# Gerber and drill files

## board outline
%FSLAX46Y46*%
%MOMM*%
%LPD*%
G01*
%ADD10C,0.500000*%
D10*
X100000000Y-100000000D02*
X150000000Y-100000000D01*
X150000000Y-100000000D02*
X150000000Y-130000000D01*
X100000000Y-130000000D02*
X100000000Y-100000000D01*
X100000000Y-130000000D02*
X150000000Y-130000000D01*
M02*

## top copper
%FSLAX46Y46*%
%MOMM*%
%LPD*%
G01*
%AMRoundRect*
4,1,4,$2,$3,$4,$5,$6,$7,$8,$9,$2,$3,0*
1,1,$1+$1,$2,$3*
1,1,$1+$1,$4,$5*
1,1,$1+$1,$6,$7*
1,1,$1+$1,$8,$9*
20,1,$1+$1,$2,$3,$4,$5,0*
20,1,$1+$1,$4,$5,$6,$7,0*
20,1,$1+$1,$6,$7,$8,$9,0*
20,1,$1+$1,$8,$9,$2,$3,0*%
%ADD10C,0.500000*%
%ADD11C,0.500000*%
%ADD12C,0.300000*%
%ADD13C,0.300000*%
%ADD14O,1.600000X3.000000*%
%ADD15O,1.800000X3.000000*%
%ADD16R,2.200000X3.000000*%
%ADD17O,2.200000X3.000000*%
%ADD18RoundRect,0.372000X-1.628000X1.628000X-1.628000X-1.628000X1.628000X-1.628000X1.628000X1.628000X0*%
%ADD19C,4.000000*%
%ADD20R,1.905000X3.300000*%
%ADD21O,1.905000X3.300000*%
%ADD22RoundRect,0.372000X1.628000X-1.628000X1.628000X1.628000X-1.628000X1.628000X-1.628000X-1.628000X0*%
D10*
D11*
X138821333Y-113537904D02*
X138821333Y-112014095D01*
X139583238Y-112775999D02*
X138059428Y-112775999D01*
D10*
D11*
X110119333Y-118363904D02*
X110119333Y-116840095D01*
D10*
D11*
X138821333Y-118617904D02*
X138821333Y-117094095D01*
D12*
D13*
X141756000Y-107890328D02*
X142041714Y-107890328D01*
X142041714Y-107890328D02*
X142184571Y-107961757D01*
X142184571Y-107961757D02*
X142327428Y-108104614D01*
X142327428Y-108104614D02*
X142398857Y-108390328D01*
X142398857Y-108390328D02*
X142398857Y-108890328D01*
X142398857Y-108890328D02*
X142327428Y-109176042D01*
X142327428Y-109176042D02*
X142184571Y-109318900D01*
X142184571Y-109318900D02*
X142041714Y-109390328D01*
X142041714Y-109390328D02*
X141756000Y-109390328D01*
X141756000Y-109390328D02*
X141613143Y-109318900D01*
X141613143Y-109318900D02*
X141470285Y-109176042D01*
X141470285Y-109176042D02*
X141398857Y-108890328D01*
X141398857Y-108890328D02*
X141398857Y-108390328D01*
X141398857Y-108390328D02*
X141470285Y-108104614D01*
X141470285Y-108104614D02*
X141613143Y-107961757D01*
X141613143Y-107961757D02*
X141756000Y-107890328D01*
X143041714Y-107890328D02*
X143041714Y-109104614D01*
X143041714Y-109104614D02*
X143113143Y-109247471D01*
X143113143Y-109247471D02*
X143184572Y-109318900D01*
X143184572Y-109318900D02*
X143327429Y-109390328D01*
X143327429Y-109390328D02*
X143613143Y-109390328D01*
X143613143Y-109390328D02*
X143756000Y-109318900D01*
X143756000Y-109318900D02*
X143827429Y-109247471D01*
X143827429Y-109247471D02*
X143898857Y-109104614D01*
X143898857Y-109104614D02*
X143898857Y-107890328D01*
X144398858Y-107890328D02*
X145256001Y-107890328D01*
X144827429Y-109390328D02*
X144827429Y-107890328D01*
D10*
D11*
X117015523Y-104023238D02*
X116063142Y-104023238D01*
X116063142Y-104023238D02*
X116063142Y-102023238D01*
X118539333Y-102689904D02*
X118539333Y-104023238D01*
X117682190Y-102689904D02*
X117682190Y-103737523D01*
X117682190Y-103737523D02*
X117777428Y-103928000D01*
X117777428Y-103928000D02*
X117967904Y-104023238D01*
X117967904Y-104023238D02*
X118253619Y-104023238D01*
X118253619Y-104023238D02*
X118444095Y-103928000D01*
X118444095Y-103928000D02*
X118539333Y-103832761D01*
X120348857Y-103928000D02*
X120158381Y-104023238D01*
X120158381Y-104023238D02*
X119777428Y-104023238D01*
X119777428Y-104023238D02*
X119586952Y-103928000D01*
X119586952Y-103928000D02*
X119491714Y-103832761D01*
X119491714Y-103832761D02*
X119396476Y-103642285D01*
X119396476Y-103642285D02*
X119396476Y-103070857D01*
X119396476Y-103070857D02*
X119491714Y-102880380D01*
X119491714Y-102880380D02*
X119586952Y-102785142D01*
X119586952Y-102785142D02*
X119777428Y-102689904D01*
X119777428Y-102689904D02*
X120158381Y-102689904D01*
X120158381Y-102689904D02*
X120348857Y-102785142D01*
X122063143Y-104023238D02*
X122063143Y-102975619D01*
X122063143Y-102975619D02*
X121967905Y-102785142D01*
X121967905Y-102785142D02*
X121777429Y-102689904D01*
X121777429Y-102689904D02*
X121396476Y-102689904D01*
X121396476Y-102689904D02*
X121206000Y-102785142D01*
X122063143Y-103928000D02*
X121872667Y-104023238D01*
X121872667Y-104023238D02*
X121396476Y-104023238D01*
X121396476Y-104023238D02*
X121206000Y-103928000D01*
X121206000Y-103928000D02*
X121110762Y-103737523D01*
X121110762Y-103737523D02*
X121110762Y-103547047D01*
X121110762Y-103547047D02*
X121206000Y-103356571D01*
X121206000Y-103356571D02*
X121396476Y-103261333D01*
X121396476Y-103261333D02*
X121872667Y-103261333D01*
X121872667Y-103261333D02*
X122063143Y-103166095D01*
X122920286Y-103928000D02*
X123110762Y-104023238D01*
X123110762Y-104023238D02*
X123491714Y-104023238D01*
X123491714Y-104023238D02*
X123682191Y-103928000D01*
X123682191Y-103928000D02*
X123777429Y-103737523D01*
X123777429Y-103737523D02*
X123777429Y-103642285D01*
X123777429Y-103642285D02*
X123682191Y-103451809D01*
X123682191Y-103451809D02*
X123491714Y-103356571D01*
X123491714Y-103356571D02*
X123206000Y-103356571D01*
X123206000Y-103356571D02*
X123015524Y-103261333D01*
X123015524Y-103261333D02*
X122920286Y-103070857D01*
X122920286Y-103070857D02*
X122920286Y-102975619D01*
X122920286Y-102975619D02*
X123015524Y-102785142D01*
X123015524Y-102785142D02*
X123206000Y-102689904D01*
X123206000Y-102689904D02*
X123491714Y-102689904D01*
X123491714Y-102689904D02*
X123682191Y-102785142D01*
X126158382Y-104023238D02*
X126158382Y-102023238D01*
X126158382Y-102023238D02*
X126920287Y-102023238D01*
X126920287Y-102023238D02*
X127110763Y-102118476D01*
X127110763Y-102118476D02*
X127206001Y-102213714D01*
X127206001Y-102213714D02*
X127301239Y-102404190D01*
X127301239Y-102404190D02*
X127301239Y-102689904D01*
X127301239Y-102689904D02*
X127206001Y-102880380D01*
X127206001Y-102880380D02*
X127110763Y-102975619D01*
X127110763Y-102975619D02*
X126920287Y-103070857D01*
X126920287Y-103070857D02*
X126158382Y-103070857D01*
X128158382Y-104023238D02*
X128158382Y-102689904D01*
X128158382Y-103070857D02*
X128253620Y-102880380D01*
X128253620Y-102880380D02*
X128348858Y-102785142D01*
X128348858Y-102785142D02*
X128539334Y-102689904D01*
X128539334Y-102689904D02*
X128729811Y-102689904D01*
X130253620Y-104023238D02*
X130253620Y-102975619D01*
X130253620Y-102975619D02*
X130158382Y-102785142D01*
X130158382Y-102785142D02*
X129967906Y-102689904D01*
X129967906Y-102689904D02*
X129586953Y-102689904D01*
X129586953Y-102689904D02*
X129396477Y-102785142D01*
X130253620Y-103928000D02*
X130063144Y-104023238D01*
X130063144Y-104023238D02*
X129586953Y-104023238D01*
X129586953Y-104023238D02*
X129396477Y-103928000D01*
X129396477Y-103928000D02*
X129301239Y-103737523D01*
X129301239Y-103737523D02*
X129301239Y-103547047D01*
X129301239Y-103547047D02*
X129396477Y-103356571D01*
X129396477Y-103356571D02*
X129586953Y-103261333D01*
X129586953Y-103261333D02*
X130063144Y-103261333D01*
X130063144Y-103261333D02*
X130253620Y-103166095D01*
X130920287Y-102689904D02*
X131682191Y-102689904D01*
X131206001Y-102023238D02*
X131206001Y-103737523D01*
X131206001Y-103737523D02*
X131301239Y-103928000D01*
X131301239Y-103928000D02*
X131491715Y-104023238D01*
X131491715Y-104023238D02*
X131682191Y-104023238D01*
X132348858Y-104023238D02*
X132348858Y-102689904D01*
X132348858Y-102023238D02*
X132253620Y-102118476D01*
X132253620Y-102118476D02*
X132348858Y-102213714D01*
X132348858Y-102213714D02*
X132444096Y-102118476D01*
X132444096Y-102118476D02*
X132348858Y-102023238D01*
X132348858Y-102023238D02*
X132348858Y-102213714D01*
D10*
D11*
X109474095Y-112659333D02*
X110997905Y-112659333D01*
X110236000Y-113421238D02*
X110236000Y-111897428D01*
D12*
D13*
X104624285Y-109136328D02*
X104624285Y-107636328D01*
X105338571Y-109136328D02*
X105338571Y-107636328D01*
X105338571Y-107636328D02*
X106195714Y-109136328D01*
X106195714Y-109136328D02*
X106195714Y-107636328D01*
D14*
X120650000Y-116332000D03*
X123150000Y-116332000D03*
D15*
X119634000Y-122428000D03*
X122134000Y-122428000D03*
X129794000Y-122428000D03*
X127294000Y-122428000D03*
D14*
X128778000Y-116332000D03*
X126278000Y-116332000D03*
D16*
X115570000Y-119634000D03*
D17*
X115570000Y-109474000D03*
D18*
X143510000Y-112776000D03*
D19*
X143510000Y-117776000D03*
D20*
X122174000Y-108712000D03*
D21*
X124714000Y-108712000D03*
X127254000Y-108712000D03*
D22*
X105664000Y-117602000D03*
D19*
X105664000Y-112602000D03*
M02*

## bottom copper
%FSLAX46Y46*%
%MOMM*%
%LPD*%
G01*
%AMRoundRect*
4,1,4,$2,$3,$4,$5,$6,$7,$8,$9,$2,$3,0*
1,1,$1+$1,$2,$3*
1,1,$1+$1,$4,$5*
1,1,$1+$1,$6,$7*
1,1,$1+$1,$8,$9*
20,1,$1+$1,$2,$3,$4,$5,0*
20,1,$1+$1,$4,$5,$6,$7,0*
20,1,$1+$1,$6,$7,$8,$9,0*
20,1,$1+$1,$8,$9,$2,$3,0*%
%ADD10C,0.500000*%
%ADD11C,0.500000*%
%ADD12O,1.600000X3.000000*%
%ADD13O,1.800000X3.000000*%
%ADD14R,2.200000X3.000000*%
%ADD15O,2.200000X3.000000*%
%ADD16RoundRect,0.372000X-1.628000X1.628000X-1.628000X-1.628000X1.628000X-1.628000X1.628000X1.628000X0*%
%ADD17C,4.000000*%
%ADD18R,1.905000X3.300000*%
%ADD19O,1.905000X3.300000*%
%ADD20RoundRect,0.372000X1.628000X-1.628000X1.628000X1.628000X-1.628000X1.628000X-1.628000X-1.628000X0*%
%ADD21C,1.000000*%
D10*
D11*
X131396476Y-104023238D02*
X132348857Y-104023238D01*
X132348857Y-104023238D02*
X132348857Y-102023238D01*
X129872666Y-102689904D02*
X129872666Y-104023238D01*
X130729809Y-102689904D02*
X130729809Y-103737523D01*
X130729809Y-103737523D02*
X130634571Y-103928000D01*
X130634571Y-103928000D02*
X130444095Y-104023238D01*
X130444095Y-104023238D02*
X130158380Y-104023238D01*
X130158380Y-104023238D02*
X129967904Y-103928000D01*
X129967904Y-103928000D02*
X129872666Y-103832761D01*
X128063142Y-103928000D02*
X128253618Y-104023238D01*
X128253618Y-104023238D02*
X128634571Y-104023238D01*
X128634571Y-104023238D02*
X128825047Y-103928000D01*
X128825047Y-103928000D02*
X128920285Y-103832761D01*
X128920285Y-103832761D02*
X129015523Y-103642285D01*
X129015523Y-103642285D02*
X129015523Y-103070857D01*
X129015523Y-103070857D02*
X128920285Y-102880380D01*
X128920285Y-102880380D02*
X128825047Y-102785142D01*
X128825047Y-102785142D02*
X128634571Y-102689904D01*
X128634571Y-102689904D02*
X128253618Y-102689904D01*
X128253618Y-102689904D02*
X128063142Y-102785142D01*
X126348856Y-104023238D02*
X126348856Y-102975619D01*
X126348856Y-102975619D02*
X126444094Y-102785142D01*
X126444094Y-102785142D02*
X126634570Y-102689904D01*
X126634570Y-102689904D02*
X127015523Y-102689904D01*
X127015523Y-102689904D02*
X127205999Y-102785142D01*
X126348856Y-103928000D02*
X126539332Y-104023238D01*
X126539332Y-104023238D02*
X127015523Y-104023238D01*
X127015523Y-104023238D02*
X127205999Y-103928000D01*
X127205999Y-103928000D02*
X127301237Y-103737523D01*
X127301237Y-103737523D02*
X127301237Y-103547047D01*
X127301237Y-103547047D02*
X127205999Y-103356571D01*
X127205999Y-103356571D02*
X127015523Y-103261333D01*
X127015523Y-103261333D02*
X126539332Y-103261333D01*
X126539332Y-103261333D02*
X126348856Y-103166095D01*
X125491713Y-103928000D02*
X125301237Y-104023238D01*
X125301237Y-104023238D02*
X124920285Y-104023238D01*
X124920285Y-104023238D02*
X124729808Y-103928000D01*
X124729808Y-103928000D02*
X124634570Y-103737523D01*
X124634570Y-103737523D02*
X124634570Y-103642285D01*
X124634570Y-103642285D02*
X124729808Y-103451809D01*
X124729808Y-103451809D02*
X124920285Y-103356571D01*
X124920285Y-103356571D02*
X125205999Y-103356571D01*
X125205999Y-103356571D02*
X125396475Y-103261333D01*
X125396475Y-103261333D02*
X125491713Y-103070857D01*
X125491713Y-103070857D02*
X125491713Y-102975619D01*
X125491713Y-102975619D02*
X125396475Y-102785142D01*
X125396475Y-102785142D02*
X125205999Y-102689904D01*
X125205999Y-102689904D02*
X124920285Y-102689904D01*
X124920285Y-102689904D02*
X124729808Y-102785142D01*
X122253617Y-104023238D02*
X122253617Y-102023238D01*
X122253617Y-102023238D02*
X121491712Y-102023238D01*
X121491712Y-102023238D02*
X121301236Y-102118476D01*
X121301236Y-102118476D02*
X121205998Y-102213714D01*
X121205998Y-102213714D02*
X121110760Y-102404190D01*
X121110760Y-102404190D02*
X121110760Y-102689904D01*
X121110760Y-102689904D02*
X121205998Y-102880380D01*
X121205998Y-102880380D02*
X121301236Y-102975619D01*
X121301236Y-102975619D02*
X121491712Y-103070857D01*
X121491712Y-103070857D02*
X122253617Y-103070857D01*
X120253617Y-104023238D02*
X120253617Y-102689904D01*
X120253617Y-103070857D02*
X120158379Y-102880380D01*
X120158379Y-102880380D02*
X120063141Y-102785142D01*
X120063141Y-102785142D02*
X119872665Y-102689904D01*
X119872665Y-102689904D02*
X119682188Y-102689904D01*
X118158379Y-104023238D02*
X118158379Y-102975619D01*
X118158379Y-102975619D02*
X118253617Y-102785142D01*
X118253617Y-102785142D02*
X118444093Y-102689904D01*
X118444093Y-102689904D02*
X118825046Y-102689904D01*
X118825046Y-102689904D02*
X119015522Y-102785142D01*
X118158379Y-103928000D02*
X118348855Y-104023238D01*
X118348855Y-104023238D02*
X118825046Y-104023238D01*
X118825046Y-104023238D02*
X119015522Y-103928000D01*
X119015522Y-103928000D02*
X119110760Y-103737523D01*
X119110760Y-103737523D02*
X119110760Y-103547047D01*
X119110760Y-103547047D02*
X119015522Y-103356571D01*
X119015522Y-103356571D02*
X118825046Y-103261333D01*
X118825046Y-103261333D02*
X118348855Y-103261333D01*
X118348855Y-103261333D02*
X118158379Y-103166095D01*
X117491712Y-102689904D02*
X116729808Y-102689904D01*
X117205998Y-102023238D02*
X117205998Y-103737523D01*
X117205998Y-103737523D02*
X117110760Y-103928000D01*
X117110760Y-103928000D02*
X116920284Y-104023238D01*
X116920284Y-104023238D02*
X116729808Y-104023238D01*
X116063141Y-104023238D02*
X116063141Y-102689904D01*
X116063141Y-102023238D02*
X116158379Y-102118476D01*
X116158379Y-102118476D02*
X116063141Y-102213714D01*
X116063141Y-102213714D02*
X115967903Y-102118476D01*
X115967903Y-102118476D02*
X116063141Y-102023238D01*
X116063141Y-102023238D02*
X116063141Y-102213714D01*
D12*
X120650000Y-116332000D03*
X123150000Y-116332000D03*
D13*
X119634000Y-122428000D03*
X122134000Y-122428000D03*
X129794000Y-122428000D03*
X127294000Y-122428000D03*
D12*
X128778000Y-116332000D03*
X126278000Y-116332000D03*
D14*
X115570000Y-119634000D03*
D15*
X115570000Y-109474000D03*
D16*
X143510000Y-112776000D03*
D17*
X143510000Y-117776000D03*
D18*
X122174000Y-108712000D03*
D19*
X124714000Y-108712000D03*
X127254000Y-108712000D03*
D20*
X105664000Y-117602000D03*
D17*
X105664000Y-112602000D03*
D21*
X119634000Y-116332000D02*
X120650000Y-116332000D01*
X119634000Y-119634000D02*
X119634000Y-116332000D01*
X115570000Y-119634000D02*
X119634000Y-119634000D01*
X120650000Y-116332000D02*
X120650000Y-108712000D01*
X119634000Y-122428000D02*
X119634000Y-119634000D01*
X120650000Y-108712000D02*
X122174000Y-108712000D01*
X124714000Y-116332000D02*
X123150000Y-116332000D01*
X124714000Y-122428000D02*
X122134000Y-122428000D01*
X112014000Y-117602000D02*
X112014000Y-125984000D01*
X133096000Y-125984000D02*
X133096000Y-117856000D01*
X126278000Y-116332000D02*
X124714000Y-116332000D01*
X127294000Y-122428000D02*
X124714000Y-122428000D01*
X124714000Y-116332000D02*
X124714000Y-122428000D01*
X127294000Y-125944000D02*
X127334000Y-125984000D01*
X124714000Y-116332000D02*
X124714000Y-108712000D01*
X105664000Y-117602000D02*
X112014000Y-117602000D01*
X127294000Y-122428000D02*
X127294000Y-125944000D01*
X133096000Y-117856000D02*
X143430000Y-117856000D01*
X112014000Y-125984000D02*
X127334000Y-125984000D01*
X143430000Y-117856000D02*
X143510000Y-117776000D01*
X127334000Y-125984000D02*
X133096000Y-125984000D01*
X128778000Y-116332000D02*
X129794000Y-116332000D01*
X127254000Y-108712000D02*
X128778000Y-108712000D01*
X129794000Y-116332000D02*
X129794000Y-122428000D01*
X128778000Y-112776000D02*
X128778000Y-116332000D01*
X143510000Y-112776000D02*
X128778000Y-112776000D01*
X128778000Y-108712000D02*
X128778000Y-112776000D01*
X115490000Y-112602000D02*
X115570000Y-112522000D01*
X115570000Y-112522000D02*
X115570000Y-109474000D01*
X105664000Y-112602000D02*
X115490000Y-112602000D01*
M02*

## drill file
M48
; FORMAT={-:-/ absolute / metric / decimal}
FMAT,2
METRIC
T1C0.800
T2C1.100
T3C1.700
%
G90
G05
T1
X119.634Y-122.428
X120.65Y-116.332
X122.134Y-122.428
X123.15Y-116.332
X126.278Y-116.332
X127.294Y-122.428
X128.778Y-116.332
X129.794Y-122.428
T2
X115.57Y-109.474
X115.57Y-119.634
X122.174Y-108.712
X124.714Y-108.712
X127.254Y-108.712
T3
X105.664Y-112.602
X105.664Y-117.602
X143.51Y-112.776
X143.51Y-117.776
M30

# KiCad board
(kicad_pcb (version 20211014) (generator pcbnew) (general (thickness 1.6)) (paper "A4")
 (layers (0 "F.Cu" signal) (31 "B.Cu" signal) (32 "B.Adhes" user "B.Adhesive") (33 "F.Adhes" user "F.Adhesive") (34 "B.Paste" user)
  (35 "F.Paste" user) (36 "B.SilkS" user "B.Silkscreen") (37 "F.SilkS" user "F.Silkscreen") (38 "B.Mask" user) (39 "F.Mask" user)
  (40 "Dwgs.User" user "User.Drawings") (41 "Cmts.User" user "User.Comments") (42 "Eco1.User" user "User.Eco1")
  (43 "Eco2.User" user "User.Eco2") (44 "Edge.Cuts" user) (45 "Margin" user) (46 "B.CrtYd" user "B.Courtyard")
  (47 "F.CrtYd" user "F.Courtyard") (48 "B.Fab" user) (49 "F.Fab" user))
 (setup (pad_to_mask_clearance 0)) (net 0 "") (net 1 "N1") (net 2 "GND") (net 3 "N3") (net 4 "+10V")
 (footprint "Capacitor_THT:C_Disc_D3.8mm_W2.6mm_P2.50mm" (layer "F.Cu") (at 120.65 116.332)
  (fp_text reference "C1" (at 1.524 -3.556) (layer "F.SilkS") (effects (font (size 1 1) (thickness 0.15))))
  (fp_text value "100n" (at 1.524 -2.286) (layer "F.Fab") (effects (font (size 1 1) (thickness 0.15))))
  (pad "1" thru_hole oval locked (at 0 0) (size 1.6 3) (drill 0.8) (layers *.Cu *.Mask) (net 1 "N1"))
  (pad "2" thru_hole oval locked (at 2.5 0) (size 1.6 3) (drill 0.8) (layers *.Cu *.Mask) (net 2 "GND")))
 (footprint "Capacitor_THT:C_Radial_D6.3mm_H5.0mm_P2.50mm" (layer "F.Cu") (at 119.634 122.428)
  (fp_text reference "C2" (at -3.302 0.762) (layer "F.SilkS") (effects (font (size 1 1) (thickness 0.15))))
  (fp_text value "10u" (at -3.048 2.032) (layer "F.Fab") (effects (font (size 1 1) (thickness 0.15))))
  (pad "1" thru_hole oval locked (at 0 0) (size 1.8 3) (drill 0.8) (layers *.Cu *.Mask) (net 1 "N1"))
  (pad "2" thru_hole oval locked (at 2.5 0) (size 1.8 3) (drill 0.8) (layers *.Cu *.Mask) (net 2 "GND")))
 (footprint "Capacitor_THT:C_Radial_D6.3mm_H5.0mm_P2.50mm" (layer "F.Cu") (at 129.794 122.428 180)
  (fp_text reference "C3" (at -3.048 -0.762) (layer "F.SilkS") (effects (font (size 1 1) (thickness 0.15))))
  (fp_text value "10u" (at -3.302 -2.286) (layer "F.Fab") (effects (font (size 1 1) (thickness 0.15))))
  (pad "1" thru_hole oval locked (at 0 0 180) (size 1.8 3) (drill 0.8) (layers *.Cu *.Mask) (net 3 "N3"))
  (pad "2" thru_hole oval locked (at 2.5 0 180) (size 1.8 3) (drill 0.8) (layers *.Cu *.Mask) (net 2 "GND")))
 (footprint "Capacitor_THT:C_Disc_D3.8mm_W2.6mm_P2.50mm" (layer "F.Cu") (at 128.778 116.332 180)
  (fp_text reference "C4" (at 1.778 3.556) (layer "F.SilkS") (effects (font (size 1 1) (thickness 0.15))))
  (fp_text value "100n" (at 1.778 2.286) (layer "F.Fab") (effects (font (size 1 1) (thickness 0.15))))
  (pad "1" thru_hole oval locked (at 0 0 180) (size 1.6 3) (drill 0.8) (layers *.Cu *.Mask) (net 3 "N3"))
  (pad "2" thru_hole oval locked (at 2.5 0 180) (size 1.6 3) (drill 0.8) (layers *.Cu *.Mask) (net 2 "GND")))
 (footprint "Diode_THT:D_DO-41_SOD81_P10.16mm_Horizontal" (layer "F.Cu") (at 115.57 119.634 90)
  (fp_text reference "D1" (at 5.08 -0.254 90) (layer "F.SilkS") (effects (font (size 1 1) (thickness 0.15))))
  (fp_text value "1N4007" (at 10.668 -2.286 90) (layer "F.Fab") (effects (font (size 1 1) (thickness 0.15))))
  (pad "1" thru_hole rect locked (at 0 0 90) (size 3 2.2) (drill 1.1) (layers *.Cu *.Mask) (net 1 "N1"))
  (pad "2" thru_hole oval locked (at 10.16 0 90) (size 3 2.2) (drill 1.1) (layers *.Cu *.Mask) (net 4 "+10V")))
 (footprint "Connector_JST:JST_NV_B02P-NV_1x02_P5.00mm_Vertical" (layer "F.Cu") (at 143.51 112.776 -90)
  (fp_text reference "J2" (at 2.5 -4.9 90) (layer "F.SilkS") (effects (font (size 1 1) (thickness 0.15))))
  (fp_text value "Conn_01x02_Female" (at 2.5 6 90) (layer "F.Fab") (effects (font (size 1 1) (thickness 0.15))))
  (pad "1" thru_hole roundrect locked (at 0 0 270) (size 4 4) (drill 1.7) (layers *.Cu *.Mask) (roundrect_rratio 0.093) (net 3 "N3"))
  (pad "2" thru_hole circle locked (at 5 0 270) (size 4 4) (drill 1.7) (layers *.Cu *.Mask) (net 2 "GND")))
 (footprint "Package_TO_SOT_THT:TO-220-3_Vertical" (layer "F.Cu") (at 122.174 108.712)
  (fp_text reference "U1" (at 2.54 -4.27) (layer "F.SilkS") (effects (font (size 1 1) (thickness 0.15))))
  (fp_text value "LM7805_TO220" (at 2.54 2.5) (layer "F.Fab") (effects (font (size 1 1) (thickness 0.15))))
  (pad "1" thru_hole rect locked (at 0 0) (size 1.905 3.3) (drill 1.1) (layers *.Cu *.Mask) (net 1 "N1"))
  (pad "2" thru_hole oval locked (at 2.54 0) (size 1.905 3.3) (drill 1.1) (layers *.Cu *.Mask) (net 2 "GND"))
  (pad "3" thru_hole oval locked (at 5.08 0) (size 1.905 3.3) (drill 1.1) (layers *.Cu *.Mask) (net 3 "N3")))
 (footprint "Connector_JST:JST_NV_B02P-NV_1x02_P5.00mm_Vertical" (layer "F.Cu") (at 105.664 117.602 90)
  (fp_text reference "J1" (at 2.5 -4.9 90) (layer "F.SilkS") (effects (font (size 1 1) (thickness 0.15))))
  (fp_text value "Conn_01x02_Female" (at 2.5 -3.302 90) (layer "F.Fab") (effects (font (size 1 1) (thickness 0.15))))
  (pad "1" thru_hole roundrect locked (at 0 0 90) (size 4 4) (drill 1.7) (layers *.Cu *.Mask) (roundrect_rratio 0.093) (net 2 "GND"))
  (pad "2" thru_hole circle locked (at 5 0 90) (size 4 4) (drill 1.7) (layers *.Cu *.Mask) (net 4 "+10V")))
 (gr_line (start 100 100) (end 150 100) (layer "Edge.Cuts") (width 0.5))
 (gr_line (start 150 100) (end 150 130) (layer "Edge.Cuts") (width 0.5))
 (gr_line (start 100 130) (end 100 100) (layer "Edge.Cuts") (width 0.5))
 (gr_line (start 100 130) (end 150 130) (layer "Edge.Cuts") (width 0.5))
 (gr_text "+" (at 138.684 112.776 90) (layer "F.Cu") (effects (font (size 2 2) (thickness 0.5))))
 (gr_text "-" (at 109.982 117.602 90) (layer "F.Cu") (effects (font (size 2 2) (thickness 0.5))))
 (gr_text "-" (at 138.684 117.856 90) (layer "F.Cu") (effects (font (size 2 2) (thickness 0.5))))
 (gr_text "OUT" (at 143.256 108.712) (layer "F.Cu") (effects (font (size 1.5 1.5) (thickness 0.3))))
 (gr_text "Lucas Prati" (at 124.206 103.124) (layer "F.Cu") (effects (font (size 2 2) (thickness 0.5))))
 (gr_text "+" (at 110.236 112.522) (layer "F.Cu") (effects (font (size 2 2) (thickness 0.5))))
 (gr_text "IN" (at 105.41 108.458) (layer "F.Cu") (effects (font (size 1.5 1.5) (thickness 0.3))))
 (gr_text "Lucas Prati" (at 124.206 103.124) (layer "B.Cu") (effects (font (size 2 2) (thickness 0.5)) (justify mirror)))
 (segment (start 119.634 116.332) (end 120.65 116.332) (width 1) (layer "B.Cu") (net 1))
 (segment (start 119.634 119.634) (end 119.634 116.332) (width 1) (layer "B.Cu") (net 1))
 (segment (start 115.57 119.634) (end 119.634 119.634) (width 1) (layer "B.Cu") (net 1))
 (segment (start 120.65 116.332) (end 120.65 108.712) (width 1) (layer "B.Cu") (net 1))
 (segment (start 119.634 122.428) (end 119.634 119.634) (width 1) (layer "B.Cu") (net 1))
 (segment (start 120.65 108.712) (end 122.174 108.712) (width 1) (layer "B.Cu") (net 1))
 (segment (start 124.714 116.332) (end 123.15 116.332) (width 1) (layer "B.Cu") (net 2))
 (segment (start 124.714 122.428) (end 122.134 122.428) (width 1) (layer "B.Cu") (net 2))
 (segment (start 112.014 117.602) (end 112.014 125.984) (width 1) (layer "B.Cu") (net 2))
 (segment (start 133.096 125.984) (end 133.096 117.856) (width 1) (layer "B.Cu") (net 2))
 (segment (start 126.278 116.332) (end 124.714 116.332) (width 1) (layer "B.Cu") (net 2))
 (segment (start 127.294 122.428) (end 124.714 122.428) (width 1) (layer "B.Cu") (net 2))
 (segment (start 124.714 116.332) (end 124.714 122.428) (width 1) (layer "B.Cu") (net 2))
 (segment (start 127.294 125.944) (end 127.334 125.984) (width 1) (layer "B.Cu") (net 2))
 (segment (start 124.714 116.332) (end 124.714 108.712) (width 1) (layer "B.Cu") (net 2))
 (segment (start 105.664 117.602) (end 112.014 117.602) (width 1) (layer "B.Cu") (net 2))
 (segment (start 127.294 122.428) (end 127.294 125.944) (width 1) (layer "B.Cu") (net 2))
 (segment (start 133.096 117.856) (end 143.43 117.856) (width 1) (layer "B.Cu") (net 2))
 (segment (start 112.014 125.984) (end 127.334 125.984) (width 1) (layer "B.Cu") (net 2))
 (segment (start 143.43 117.856) (end 143.51 117.776) (width 1) (layer "B.Cu") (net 2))
 (segment (start 127.334 125.984) (end 133.096 125.984) (width 1) (layer "B.Cu") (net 2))
 (segment (start 128.778 116.332) (end 129.794 116.332) (width 1) (layer "B.Cu") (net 3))
 (segment (start 127.254 108.712) (end 128.778 108.712) (width 1) (layer "B.Cu") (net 3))
 (segment (start 129.794 116.332) (end 129.794 122.428) (width 1) (layer "B.Cu") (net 3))
 (segment (start 128.778 112.776) (end 128.778 116.332) (width 1) (layer "B.Cu") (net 3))
 (segment (start 143.51 112.776) (end 128.778 112.776) (width 1) (layer "B.Cu") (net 3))
 (segment (start 128.778 108.712) (end 128.778 112.776) (width 1) (layer "B.Cu") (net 3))
 (segment (start 115.49 112.602) (end 115.57 112.522) (width 1) (layer "B.Cu") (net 4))
 (segment (start 115.57 112.522) (end 115.57 109.474) (width 1) (layer "B.Cu") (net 4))
 (segment (start 105.664 112.602) (end 115.49 112.602) (width 1) (layer "B.Cu") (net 4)))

